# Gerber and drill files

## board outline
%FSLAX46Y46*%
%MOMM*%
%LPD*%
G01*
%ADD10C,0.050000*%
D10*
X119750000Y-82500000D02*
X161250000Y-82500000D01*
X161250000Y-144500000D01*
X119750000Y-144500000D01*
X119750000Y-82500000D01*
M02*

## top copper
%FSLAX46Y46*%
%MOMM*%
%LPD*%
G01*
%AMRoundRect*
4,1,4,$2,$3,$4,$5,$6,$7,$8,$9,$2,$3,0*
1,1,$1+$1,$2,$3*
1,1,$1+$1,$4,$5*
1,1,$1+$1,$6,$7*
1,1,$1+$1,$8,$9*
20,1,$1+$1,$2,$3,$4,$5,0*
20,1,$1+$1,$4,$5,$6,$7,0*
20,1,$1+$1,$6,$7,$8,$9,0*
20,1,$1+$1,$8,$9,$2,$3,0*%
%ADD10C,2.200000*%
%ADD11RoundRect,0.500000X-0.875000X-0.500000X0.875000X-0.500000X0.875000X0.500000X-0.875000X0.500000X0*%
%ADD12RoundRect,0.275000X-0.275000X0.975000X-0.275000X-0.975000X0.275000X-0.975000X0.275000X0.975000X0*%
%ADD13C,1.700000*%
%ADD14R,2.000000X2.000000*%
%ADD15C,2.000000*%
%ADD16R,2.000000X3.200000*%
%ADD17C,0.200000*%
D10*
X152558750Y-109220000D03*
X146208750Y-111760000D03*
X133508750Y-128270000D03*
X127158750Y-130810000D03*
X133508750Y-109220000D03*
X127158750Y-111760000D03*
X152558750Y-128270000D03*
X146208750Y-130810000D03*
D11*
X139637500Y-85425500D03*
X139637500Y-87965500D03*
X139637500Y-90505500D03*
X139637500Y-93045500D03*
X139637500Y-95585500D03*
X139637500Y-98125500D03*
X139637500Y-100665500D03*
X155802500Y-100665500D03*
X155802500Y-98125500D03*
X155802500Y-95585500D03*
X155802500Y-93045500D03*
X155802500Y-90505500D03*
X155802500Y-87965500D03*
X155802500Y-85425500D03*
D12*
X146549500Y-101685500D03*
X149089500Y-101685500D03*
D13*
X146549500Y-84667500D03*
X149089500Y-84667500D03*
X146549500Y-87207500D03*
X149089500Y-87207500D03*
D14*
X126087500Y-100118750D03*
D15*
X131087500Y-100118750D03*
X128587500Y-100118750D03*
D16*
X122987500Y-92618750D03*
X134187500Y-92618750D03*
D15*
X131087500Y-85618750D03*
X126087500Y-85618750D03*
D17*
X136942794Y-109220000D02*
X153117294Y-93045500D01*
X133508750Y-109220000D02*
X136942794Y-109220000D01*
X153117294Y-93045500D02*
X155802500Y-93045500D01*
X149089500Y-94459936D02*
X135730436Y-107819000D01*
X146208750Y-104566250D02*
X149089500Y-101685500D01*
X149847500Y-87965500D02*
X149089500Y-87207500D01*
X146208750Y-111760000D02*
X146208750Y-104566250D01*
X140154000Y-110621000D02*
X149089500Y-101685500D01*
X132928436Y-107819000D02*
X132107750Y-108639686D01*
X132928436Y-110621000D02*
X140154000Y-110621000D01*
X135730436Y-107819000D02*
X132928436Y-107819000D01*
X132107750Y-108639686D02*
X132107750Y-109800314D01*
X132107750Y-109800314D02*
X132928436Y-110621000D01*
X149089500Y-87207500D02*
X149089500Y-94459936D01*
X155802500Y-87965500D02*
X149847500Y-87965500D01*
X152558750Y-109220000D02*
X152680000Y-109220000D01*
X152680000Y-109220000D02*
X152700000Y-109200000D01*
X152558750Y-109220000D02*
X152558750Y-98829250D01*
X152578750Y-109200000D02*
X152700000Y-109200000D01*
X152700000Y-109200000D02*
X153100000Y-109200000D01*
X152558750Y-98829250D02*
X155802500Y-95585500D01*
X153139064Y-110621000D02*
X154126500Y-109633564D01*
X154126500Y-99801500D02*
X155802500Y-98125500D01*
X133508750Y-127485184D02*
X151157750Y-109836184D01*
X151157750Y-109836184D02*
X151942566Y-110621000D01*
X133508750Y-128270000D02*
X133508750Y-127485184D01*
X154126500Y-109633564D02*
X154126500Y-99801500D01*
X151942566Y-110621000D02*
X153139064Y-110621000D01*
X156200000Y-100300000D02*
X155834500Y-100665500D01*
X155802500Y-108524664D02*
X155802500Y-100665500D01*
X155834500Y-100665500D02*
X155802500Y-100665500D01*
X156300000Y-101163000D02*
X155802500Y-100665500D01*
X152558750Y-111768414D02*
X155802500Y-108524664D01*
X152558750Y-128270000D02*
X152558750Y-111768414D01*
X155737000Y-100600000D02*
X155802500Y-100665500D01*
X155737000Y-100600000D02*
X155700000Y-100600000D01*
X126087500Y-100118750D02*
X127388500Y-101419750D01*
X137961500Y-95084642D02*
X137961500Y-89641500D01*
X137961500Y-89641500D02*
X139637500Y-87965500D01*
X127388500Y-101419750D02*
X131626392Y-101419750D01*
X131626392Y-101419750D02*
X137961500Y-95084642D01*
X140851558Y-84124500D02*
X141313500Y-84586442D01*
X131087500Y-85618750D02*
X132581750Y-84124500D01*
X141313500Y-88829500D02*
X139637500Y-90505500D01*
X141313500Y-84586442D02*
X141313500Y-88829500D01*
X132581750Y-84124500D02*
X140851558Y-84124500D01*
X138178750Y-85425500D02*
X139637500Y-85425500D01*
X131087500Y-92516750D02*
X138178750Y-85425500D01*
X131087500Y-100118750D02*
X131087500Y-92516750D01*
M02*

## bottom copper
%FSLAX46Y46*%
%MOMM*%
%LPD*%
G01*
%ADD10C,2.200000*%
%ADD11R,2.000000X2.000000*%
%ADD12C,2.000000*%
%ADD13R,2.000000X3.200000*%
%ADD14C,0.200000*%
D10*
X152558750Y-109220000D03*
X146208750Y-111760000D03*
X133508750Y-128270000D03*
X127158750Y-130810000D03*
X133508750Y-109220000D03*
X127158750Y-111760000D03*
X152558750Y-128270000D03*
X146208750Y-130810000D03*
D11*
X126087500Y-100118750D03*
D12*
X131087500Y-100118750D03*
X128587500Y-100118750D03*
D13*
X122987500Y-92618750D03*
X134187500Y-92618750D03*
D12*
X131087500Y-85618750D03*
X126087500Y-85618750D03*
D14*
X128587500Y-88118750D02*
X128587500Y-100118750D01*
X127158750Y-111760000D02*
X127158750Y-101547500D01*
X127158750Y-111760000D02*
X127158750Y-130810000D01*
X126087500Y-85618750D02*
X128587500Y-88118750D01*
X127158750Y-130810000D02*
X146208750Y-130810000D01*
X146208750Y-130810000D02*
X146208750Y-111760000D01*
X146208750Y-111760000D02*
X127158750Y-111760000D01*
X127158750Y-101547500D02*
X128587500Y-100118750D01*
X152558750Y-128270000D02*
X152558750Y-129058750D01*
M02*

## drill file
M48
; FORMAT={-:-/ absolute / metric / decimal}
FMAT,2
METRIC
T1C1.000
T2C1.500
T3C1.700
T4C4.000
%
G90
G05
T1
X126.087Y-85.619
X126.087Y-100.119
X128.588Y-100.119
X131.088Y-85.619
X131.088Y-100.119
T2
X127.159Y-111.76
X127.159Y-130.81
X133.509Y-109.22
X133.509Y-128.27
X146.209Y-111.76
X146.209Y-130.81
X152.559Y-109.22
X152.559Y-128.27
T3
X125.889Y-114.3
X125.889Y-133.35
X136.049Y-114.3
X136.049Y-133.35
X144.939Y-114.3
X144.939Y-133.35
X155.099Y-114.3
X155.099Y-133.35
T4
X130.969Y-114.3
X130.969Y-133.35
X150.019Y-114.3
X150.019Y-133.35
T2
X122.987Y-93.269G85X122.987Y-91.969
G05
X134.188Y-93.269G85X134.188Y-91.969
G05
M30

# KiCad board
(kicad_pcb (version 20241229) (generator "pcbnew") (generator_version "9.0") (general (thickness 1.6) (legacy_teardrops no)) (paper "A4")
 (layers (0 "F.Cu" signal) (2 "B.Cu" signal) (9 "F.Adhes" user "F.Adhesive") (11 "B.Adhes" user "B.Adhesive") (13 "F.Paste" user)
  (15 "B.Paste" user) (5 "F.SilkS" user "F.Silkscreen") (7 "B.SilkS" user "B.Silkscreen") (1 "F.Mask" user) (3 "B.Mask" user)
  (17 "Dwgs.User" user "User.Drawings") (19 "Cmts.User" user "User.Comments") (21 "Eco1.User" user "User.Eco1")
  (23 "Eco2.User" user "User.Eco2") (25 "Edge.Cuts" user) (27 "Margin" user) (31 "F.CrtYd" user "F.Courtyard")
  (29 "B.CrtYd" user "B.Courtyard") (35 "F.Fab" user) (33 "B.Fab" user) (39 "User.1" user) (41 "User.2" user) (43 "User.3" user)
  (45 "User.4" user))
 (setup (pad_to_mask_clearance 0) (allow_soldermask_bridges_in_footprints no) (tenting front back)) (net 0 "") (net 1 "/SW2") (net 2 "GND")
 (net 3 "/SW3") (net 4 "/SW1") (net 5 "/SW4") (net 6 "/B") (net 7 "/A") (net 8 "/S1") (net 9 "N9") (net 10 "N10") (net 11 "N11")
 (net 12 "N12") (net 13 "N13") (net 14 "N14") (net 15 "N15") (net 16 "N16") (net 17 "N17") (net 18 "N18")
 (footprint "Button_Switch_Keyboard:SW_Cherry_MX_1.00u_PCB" (layer "F.Cu") (at 152.55875 109.22)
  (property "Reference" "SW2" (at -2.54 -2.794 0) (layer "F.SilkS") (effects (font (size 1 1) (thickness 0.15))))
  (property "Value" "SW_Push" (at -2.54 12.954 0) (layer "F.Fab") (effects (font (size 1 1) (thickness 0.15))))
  (pad "" np_thru_hole circle (at -7.62 5.08) (size 1.7 1.7) (drill 1.7) (layers "*.Cu" "*.Mask"))
  (pad "" np_thru_hole circle (at -2.54 5.08) (size 4 4) (drill 4) (layers "*.Cu" "*.Mask"))
  (pad "" np_thru_hole circle (at 2.54 5.08) (size 1.7 1.7) (drill 1.7) (layers "*.Cu" "*.Mask"))
  (pad "1" thru_hole circle (at 0 0) (size 2.2 2.2) (drill 1.5) (layers "*.Cu" "*.Mask") (remove_unused_layers no) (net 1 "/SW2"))
  (pad "2" thru_hole circle (at -6.35 2.54) (size 2.2 2.2) (drill 1.5) (layers "*.Cu" "*.Mask") (remove_unused_layers no) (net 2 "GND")))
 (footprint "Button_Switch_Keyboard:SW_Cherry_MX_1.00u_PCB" (layer "F.Cu") (at 133.50875 128.27)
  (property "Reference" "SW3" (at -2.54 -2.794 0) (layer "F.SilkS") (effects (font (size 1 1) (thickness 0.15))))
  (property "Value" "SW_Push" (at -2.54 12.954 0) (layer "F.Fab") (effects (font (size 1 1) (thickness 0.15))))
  (pad "" np_thru_hole circle (at -7.62 5.08) (size 1.7 1.7) (drill 1.7) (layers "*.Cu" "*.Mask"))
  (pad "" np_thru_hole circle (at -2.54 5.08) (size 4 4) (drill 4) (layers "*.Cu" "*.Mask"))
  (pad "" np_thru_hole circle (at 2.54 5.08) (size 1.7 1.7) (drill 1.7) (layers "*.Cu" "*.Mask"))
  (pad "1" thru_hole circle (at 0 0) (size 2.2 2.2) (drill 1.5) (layers "*.Cu" "*.Mask") (remove_unused_layers no) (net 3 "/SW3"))
  (pad "2" thru_hole circle (at -6.35 2.54) (size 2.2 2.2) (drill 1.5) (layers "*.Cu" "*.Mask") (remove_unused_layers no) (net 2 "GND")))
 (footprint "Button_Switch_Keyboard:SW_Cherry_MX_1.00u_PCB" (layer "F.Cu") (at 133.50875 109.22)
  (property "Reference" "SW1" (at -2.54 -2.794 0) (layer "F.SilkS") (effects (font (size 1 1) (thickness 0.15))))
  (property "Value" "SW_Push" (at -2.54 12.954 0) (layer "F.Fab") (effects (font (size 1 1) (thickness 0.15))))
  (pad "" np_thru_hole circle (at -7.62 5.08) (size 1.7 1.7) (drill 1.7) (layers "*.Cu" "*.Mask"))
  (pad "" np_thru_hole circle (at -2.54 5.08) (size 4 4) (drill 4) (layers "*.Cu" "*.Mask"))
  (pad "" np_thru_hole circle (at 2.54 5.08) (size 1.7 1.7) (drill 1.7) (layers "*.Cu" "*.Mask"))
  (pad "1" thru_hole circle (at 0 0) (size 2.2 2.2) (drill 1.5) (layers "*.Cu" "*.Mask") (remove_unused_layers no) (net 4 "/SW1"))
  (pad "2" thru_hole circle (at -6.35 2.54) (size 2.2 2.2) (drill 1.5) (layers "*.Cu" "*.Mask") (remove_unused_layers no) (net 2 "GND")))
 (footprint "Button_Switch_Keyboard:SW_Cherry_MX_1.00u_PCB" (layer "F.Cu") (at 152.55875 128.27)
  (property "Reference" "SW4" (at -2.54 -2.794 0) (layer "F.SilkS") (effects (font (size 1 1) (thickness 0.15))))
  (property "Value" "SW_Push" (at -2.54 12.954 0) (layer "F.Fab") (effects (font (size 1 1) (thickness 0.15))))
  (pad "" np_thru_hole circle (at -7.62 5.08) (size 1.7 1.7) (drill 1.7) (layers "*.Cu" "*.Mask"))
  (pad "" np_thru_hole circle (at -2.54 5.08) (size 4 4) (drill 4) (layers "*.Cu" "*.Mask"))
  (pad "" np_thru_hole circle (at 2.54 5.08) (size 1.7 1.7) (drill 1.7) (layers "*.Cu" "*.Mask"))
  (pad "1" thru_hole circle (at 0 0) (size 2.2 2.2) (drill 1.5) (layers "*.Cu" "*.Mask") (remove_unused_layers no) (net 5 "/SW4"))
  (pad "2" thru_hole circle (at -6.35 2.54) (size 2.2 2.2) (drill 1.5) (layers "*.Cu" "*.Mask") (remove_unused_layers no) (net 2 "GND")))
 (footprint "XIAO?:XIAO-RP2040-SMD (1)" (layer "F.Cu") (at 147.6375 93.0455)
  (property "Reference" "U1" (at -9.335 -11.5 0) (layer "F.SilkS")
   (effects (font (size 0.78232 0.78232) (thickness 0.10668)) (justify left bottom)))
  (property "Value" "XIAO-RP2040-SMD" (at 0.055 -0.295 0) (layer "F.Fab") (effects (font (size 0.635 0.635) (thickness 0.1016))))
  (pad "1" smd roundrect (at -8 -7.62) (size 2.75 2) (layers "F.Cu" "F.Mask" "F.Paste") (roundrect_rratio 0.25) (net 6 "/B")
   (solder_mask_margin 0.0508) (thermal_bridge_angle 45))
  (pad "2" smd roundrect (at -8 -5.08) (size 2.75 2) (layers "F.Cu" "F.Mask" "F.Paste") (roundrect_rratio 0.25) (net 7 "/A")
   (solder_mask_margin 0.0508) (thermal_bridge_angle 45))
  (pad "3" smd roundrect (at -8 -2.54) (size 2.75 2) (layers "F.Cu" "F.Mask" "F.Paste") (roundrect_rratio 0.25) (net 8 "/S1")
   (solder_mask_margin 0.0508) (thermal_bridge_angle 45))
  (pad "4" smd roundrect (at -8 0) (size 2.75 2) (layers "F.Cu" "F.Mask" "F.Paste") (roundrect_rratio 0.25) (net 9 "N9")
   (solder_mask_margin 0.0508) (thermal_bridge_angle 45))
  (pad "5" smd roundrect (at -8 2.54) (size 2.75 2) (layers "F.Cu" "F.Mask" "F.Paste") (roundrect_rratio 0.25) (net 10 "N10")
   (solder_mask_margin 0.0508) (thermal_bridge_angle 45))
  (pad "6" smd roundrect (at -8 5.08) (size 2.75 2) (layers "F.Cu" "F.Mask" "F.Paste") (roundrect_rratio 0.25) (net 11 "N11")
   (solder_mask_margin 0.0508) (thermal_bridge_angle 45))
  (pad "7" smd roundrect (at -8 7.62) (size 2.75 2) (layers "F.Cu" "F.Mask" "F.Paste") (roundrect_rratio 0.25) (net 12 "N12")
   (solder_mask_margin 0.0508) (thermal_bridge_angle 45))
  (pad "8" smd roundrect (at 8.165 7.62) (size 2.75 2) (layers "F.Cu" "F.Mask" "F.Paste") (roundrect_rratio 0.25) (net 5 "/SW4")
   (solder_mask_margin 0.0508) (thermal_bridge_angle 45))
  (pad "9" smd roundrect (at 8.165 5.08) (size 2.75 2) (layers "F.Cu" "F.Mask" "F.Paste") (roundrect_rratio 0.25) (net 3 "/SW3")
   (solder_mask_margin 0.0508) (thermal_bridge_angle 45))
  (pad "10" smd roundrect (at 8.165 2.54) (size 2.75 2) (layers "F.Cu" "F.Mask" "F.Paste") (roundrect_rratio 0.25) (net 1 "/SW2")
   (solder_mask_margin 0.0508) (thermal_bridge_angle 45))
  (pad "11" smd roundrect (at 8.165 0) (size 2.75 2) (layers "F.Cu" "F.Mask" "F.Paste") (roundrect_rratio 0.25) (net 4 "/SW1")
   (solder_mask_margin 0.0508) (thermal_bridge_angle 45))
  (pad "12" smd roundrect (at 8.165 -2.54) (size 2.75 2) (layers "F.Cu" "F.Mask" "F.Paste") (roundrect_rratio 0.25) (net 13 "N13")
   (solder_mask_margin 0.0508) (thermal_bridge_angle 45))
  (pad "13" smd roundrect (at 8.165 -5.08) (size 2.75 2) (layers "F.Cu" "F.Mask" "F.Paste") (roundrect_rratio 0.25) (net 2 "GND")
   (solder_mask_margin 0.0508) (thermal_bridge_angle 45))
  (pad "14" smd roundrect (at 8.165 -7.62) (size 2.75 2) (layers "F.Cu" "F.Mask" "F.Paste") (roundrect_rratio 0.25) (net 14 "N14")
   (solder_mask_margin 0.0508) (thermal_bridge_angle 45))
  (pad "15" smd roundrect (at -1.088 8.64 270) (size 2.5 1.1) (layers "F.Cu" "F.Mask" "F.Paste") (roundrect_rratio 0.25) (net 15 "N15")
   (thermal_bridge_angle 45))
  (pad "16" smd roundrect (at 1.452 8.64 270) (size 2.5 1.1) (layers "F.Cu" "F.Mask" "F.Paste") (roundrect_rratio 0.25) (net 2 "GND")
   (thermal_bridge_angle 45))
  (pad "17" smd circle (at -1.088 -8.378) (size 1.7 1.7) (layers "F.Cu" "F.Mask" "F.Paste") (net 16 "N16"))
  (pad "18" smd circle (at 1.452 -8.378) (size 1.7 1.7) (layers "F.Cu" "F.Mask" "F.Paste") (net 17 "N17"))
  (pad "19" smd circle (at -1.088 -5.838) (size 1.7 1.7) (layers "F.Cu" "F.Mask" "F.Paste") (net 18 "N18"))
  (pad "20" smd circle (at 1.452 -5.838) (size 1.7 1.7) (layers "F.Cu" "F.Mask" "F.Paste") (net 2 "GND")))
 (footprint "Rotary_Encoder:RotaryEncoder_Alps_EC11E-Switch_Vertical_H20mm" (layer "F.Cu") (at 126.0875 100.11875 90)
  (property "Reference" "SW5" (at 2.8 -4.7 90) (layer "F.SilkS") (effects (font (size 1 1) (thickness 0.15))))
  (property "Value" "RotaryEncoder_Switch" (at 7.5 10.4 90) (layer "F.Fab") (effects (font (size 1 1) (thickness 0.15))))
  (pad "A" thru_hole rect (at 0 0 90) (size 2 2) (drill 1) (layers "*.Cu" "*.Mask") (remove_unused_layers no) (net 7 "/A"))
  (pad "B" thru_hole circle (at 0 5 90) (size 2 2) (drill 1) (layers "*.Cu" "*.Mask") (remove_unused_layers no) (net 6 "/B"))
  (pad "C" thru_hole circle (at 0 2.5 90) (size 2 2) (drill 1) (layers "*.Cu" "*.Mask") (remove_unused_layers no) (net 2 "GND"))
  (pad "MP" thru_hole rect (at 7.5 -3.1 90) (size 3.2 2) (drill oval 2.8 1.5) (layers "*.Cu" "*.Mask") (remove_unused_layers no))
  (pad "MP" thru_hole rect (at 7.5 8.1 90) (size 3.2 2) (drill oval 2.8 1.5) (layers "*.Cu" "*.Mask") (remove_unused_layers no))
  (pad "S1" thru_hole circle (at 14.5 5 90) (size 2 2) (drill 1) (layers "*.Cu" "*.Mask") (remove_unused_layers no) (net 8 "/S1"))
  (pad "S2" thru_hole circle (at 14.5 0 90) (size 2 2) (drill 1) (layers "*.Cu" "*.Mask") (remove_unused_layers no) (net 2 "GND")))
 (gr_rect (start 119.75 82.5) (end 161.25 144.5) (stroke (width 0.05) (type default)) (fill no) (layer "Edge.Cuts"))
 (segment (start 136.942794 109.22) (end 153.117294 93.0455) (width 0.2) (layer "F.Cu") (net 4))
 (segment (start 133.50875 109.22) (end 136.942794 109.22) (width 0.2) (layer "F.Cu") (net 4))
 (segment (start 153.117294 93.0455) (end 155.8025 93.0455) (width 0.2) (layer "F.Cu") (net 4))
 (segment (start 149.0895 94.459936) (end 135.730436 107.819) (width 0.2) (layer "F.Cu") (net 2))
 (segment (start 146.20875 104.56625) (end 149.0895 101.6855) (width 0.2) (layer "F.Cu") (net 2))
 (segment (start 149.8475 87.9655) (end 149.0895 87.2075) (width 0.2) (layer "F.Cu") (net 2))
 (segment (start 146.20875 111.76) (end 146.20875 104.56625) (width 0.2) (layer "F.Cu") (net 2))
 (segment (start 140.154 110.621) (end 149.0895 101.6855) (width 0.2) (layer "F.Cu") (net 2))
 (segment (start 132.928436 107.819) (end 132.10775 108.639686) (width 0.2) (layer "F.Cu") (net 2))
 (segment (start 132.928436 110.621) (end 140.154 110.621) (width 0.2) (layer "F.Cu") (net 2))
 (segment (start 135.730436 107.819) (end 132.928436 107.819) (width 0.2) (layer "F.Cu") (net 2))
 (segment (start 132.10775 108.639686) (end 132.10775 109.800314) (width 0.2) (layer "F.Cu") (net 2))
 (segment (start 132.10775 109.800314) (end 132.928436 110.621) (width 0.2) (layer "F.Cu") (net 2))
 (segment (start 149.0895 87.2075) (end 149.0895 94.459936) (width 0.2) (layer "F.Cu") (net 2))
 (segment (start 155.8025 87.9655) (end 149.8475 87.9655) (width 0.2) (layer "F.Cu") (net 2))
 (segment (start 128.5875 88.11875) (end 128.5875 100.11875) (width 0.2) (layer "B.Cu") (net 2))
 (segment (start 127.15875 111.76) (end 127.15875 101.5475) (width 0.2) (layer "B.Cu") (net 2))
 (segment (start 127.15875 111.76) (end 127.15875 130.81) (width 0.2) (layer "B.Cu") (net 2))
 (segment (start 126.0875 85.61875) (end 128.5875 88.11875) (width 0.2) (layer "B.Cu") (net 2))
 (segment (start 127.15875 130.81) (end 146.20875 130.81) (width 0.2) (layer "B.Cu") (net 2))
 (segment (start 146.20875 130.81) (end 146.20875 111.76) (width 0.2) (layer "B.Cu") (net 2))
 (segment (start 146.20875 111.76) (end 127.15875 111.76) (width 0.2) (layer "B.Cu") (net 2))
 (segment (start 127.15875 101.5475) (end 128.5875 100.11875) (width 0.2) (layer "B.Cu") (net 2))
 (segment (start 152.55875 109.22) (end 152.68 109.22) (width 0.2) (layer "F.Cu") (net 1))
 (segment (start 152.68 109.22) (end 152.7 109.2) (width 0.2) (layer "F.Cu") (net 1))
 (segment (start 152.55875 109.22) (end 152.55875 98.82925) (width 0.2) (layer "F.Cu") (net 1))
 (segment (start 152.57875 109.2) (end 152.7 109.2) (width 0.2) (layer "F.Cu") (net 1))
 (segment (start 152.7 109.2) (end 153.1 109.2) (width 0.2) (layer "F.Cu") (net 1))
 (segment (start 152.55875 98.82925) (end 155.8025 95.5855) (width 0.2) (layer "F.Cu") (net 1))
 (segment (start 153.139064 110.621) (end 154.1265 109.633564) (width 0.2) (layer "F.Cu") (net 3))
 (segment (start 154.1265 99.8015) (end 155.8025 98.1255) (width 0.2) (layer "F.Cu") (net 3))
 (segment (start 133.50875 127.485184) (end 151.15775 109.836184) (width 0.2) (layer "F.Cu") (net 3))
 (segment (start 151.15775 109.836184) (end 151.942566 110.621) (width 0.2) (layer "F.Cu") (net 3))
 (segment (start 133.50875 128.27) (end 133.50875 127.485184) (width 0.2) (layer "F.Cu") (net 3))
 (segment (start 154.1265 109.633564) (end 154.1265 99.8015) (width 0.2) (layer "F.Cu") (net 3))
 (segment (start 151.942566 110.621) (end 153.139064 110.621) (width 0.2) (layer "F.Cu") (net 3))
 (segment (start 156.2 100.3) (end 155.8345 100.6655) (width 0.2) (layer "F.Cu") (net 5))
 (segment (start 155.8025 108.524664) (end 155.8025 100.6655) (width 0.2) (layer "F.Cu") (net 5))
 (segment (start 155.8345 100.6655) (end 155.8025 100.6655) (width 0.2) (layer "F.Cu") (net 5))
 (segment (start 156.3 101.163) (end 155.8025 100.6655) (width 0.2) (layer "F.Cu") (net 5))
 (segment (start 152.55875 111.768414) (end 155.8025 108.524664) (width 0.2) (layer "F.Cu") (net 5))
 (segment (start 152.55875 128.27) (end 152.55875 111.768414) (width 0.2) (layer "F.Cu") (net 5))
 (segment (start 155.737 100.6) (end 155.8025 100.6655) (width 0.2) (layer "F.Cu") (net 5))
 (segment (start 155.737 100.6) (end 155.7 100.6) (width 0.2) (layer "F.Cu") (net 5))
 (segment (start 152.55875 128.27) (end 152.55875 129.05875) (width 0.2) (layer "B.Cu") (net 5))
 (segment (start 126.0875 100.11875) (end 127.3885 101.41975) (width 0.2) (layer "F.Cu") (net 7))
 (segment (start 137.9615 95.084642) (end 137.9615 89.6415) (width 0.2) (layer "F.Cu") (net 7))
 (segment (start 137.9615 89.6415) (end 139.6375 87.9655) (width 0.2) (layer "F.Cu") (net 7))
 (segment (start 127.3885 101.41975) (end 131.626392 101.41975) (width 0.2) (layer "F.Cu") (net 7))
 (segment (start 131.626392 101.41975) (end 137.9615 95.084642) (width 0.2) (layer "F.Cu") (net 7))
 (segment (start 140.851558 84.1245) (end 141.3135 84.586442) (width 0.2) (layer "F.Cu") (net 8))
 (segment (start 131.0875 85.61875) (end 132.58175 84.1245) (width 0.2) (layer "F.Cu") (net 8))
 (segment (start 141.3135 88.8295) (end 139.6375 90.5055) (width 0.2) (layer "F.Cu") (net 8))
 (segment (start 141.3135 84.586442) (end 141.3135 88.8295) (width 0.2) (layer "F.Cu") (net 8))
 (segment (start 132.58175 84.1245) (end 140.851558 84.1245) (width 0.2) (layer "F.Cu") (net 8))
 (segment (start 138.17875 85.4255) (end 139.6375 85.4255) (width 0.2) (layer "F.Cu") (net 6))
 (segment (start 131.0875 92.51675) (end 138.17875 85.4255) (width 0.2) (layer "F.Cu") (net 6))
 (segment (start 131.0875 100.11875) (end 131.0875 92.51675) (width 0.2) (layer "F.Cu") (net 6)))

